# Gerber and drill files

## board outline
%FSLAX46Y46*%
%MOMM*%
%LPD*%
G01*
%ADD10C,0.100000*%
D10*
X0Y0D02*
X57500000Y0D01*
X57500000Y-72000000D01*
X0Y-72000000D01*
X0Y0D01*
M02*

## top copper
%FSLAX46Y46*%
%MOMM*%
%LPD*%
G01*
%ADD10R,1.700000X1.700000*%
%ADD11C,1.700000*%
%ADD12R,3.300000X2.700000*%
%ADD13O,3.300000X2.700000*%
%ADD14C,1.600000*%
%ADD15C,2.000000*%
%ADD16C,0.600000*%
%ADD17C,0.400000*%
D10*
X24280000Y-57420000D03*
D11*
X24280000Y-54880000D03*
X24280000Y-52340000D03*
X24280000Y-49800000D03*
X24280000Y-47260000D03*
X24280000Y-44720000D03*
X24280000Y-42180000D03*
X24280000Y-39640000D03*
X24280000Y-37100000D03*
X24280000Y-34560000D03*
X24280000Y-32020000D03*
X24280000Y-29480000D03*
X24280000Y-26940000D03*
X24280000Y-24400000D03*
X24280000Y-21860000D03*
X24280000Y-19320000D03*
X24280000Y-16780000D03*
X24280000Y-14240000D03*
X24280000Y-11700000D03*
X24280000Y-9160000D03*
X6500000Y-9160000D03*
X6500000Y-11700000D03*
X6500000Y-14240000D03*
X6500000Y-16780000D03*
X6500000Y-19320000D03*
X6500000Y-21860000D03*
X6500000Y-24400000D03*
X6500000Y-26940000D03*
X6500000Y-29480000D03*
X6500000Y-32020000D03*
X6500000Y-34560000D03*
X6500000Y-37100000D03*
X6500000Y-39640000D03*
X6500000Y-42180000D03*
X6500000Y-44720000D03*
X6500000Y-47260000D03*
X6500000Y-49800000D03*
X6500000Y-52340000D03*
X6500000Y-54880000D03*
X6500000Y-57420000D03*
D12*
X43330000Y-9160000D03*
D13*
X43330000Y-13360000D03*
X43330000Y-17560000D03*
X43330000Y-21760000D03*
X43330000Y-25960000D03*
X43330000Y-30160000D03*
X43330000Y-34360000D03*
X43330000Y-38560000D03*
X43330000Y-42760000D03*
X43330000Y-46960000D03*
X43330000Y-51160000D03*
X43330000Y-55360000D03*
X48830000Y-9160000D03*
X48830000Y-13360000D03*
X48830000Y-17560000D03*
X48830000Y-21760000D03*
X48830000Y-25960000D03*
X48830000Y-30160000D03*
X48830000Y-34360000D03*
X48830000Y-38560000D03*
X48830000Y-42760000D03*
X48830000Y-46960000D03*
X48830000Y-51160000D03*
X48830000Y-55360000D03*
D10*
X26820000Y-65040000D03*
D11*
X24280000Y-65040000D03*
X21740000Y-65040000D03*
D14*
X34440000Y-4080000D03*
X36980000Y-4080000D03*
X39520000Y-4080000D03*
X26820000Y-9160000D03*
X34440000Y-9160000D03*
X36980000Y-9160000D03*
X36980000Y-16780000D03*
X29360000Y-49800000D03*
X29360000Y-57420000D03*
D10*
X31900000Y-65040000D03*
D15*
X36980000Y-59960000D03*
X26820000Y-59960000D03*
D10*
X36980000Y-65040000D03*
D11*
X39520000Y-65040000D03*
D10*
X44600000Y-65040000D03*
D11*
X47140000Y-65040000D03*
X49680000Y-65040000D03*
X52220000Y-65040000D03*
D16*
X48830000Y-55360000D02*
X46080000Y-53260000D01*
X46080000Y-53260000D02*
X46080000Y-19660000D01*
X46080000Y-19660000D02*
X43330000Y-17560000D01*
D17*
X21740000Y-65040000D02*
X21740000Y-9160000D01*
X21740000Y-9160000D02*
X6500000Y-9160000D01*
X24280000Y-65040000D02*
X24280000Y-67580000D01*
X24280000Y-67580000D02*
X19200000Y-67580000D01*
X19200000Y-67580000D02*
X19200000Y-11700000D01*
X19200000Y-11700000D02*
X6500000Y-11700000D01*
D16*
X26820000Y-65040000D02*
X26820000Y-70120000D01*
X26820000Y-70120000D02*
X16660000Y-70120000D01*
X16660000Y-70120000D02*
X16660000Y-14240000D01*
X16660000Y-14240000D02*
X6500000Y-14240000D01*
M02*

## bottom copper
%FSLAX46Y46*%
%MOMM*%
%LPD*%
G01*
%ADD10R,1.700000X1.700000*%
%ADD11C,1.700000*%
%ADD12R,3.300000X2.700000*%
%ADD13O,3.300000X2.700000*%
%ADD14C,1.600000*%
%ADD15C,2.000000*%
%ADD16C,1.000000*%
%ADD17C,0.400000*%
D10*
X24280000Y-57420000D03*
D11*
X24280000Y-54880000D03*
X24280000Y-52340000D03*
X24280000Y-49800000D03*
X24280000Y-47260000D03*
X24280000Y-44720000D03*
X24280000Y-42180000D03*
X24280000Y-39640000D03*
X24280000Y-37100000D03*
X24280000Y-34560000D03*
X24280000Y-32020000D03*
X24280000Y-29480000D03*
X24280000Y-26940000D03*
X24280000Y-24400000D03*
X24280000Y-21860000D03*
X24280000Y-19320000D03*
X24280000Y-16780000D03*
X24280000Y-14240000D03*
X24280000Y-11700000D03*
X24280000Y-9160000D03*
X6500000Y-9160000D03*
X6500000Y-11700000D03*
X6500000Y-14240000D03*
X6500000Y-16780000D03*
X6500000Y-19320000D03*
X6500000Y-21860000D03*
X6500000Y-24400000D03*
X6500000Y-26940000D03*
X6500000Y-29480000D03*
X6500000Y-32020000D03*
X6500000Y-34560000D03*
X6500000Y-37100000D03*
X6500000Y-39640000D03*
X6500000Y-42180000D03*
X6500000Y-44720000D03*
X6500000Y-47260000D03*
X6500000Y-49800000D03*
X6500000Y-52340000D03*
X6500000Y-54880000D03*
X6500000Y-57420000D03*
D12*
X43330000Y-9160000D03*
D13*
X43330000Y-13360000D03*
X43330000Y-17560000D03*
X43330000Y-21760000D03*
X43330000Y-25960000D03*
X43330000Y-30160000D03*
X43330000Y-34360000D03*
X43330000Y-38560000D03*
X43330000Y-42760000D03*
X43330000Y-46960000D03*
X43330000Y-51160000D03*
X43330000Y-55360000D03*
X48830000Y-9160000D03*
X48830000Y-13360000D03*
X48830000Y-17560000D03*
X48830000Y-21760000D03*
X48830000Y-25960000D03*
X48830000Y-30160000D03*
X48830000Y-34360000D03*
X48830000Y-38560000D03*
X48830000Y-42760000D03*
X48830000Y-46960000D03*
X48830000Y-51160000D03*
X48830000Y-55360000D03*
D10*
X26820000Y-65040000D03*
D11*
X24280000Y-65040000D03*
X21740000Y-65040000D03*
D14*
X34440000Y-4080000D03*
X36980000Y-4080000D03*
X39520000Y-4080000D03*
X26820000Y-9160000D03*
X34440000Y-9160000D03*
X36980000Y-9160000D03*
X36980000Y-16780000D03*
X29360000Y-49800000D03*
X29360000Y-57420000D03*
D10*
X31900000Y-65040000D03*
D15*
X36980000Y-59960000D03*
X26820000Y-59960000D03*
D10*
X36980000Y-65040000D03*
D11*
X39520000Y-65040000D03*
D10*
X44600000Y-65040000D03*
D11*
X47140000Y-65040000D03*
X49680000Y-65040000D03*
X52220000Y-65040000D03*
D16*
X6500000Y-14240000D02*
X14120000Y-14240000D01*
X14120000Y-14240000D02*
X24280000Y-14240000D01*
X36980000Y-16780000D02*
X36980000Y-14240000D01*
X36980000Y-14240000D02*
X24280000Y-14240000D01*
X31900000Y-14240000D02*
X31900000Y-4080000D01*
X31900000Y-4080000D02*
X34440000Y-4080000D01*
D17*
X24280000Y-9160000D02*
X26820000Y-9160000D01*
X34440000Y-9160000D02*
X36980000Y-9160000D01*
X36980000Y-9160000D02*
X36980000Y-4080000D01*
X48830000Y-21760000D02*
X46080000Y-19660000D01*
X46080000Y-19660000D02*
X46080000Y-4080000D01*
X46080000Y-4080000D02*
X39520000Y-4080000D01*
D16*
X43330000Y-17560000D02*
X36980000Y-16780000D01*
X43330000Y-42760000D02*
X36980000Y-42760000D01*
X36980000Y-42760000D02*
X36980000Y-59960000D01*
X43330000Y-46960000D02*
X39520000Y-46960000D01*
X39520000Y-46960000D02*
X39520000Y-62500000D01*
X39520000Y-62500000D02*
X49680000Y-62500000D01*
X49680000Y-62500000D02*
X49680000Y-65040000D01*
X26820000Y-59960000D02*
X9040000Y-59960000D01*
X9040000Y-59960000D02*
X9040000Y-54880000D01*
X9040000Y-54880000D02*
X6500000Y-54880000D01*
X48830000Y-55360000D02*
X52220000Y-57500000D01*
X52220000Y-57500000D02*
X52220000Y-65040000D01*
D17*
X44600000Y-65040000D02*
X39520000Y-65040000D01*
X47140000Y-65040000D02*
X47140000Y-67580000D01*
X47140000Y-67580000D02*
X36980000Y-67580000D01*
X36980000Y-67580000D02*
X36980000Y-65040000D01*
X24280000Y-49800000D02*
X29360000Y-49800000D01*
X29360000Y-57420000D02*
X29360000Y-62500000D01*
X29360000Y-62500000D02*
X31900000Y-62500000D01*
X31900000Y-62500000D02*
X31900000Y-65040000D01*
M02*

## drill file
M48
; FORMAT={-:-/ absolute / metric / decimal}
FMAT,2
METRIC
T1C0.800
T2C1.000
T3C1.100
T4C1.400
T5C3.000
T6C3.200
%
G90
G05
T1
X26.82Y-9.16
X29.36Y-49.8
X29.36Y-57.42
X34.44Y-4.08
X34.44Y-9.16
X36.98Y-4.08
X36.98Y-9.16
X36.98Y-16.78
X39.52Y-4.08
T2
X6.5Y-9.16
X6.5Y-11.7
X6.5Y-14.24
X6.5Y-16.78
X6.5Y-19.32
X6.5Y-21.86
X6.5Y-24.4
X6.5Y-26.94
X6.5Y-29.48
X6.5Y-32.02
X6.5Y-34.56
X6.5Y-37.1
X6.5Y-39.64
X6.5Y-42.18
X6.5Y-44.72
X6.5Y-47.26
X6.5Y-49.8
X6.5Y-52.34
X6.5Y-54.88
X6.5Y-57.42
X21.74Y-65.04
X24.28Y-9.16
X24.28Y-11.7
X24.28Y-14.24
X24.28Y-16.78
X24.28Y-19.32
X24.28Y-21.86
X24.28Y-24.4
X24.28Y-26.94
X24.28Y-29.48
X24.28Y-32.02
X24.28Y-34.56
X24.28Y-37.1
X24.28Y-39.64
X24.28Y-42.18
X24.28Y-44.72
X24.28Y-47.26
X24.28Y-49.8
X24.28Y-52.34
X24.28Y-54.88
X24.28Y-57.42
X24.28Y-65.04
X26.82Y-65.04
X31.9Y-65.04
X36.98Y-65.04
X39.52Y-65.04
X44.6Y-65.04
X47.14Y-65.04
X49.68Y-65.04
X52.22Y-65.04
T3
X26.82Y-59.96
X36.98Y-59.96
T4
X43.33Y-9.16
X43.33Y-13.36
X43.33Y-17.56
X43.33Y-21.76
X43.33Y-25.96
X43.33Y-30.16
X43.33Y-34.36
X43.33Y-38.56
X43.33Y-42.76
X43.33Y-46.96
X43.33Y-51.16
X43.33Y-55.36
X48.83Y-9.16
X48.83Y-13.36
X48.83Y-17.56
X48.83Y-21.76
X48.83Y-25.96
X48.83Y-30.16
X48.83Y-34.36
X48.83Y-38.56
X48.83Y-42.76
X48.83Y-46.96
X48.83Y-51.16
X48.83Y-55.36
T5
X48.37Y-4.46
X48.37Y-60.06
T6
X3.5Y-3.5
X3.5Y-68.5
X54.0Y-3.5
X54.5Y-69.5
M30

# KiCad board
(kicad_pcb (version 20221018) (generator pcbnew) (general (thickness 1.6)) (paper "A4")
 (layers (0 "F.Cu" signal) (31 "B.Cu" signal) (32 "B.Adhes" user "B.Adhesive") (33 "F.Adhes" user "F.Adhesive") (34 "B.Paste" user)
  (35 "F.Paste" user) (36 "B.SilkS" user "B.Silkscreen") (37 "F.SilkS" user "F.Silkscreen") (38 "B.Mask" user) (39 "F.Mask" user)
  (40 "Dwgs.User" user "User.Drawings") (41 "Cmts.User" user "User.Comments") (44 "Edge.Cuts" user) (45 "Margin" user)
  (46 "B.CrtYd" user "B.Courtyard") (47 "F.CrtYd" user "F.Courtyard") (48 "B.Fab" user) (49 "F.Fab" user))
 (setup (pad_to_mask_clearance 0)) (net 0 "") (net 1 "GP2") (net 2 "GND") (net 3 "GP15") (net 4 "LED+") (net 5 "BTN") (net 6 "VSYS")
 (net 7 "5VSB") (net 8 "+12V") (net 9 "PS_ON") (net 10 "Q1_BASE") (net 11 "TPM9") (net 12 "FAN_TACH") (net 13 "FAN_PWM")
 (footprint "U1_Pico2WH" (layer "F.Cu") (at 15.390 33.290) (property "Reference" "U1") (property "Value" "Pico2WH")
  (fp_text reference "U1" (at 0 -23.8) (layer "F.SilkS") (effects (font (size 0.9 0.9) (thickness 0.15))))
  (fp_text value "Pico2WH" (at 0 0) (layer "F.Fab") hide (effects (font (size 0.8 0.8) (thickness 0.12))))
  (pad "1" thru_hole rect (at 8.890 24.130) (size 1.7 1.7) (drill 1.0) (layers "*.Cu" "*.Mask"))
  (pad "2" thru_hole circle (at 8.890 21.590) (size 1.7 1.7) (drill 1.0) (layers "*.Cu" "*.Mask"))
  (pad "3" thru_hole circle (at 8.890 19.050) (size 1.7 1.7) (drill 1.0) (layers "*.Cu" "*.Mask"))
  (pad "4" thru_hole circle (at 8.890 16.510) (size 1.7 1.7) (drill 1.0) (layers "*.Cu" "*.Mask") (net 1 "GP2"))
  (pad "5" thru_hole circle (at 8.890 13.970) (size 1.7 1.7) (drill 1.0) (layers "*.Cu" "*.Mask"))
  (pad "6" thru_hole circle (at 8.890 11.430) (size 1.7 1.7) (drill 1.0) (layers "*.Cu" "*.Mask"))
  (pad "7" thru_hole circle (at 8.890 8.890) (size 1.7 1.7) (drill 1.0) (layers "*.Cu" "*.Mask"))
  (pad "8" thru_hole circle (at 8.890 6.350) (size 1.7 1.7) (drill 1.0) (layers "*.Cu" "*.Mask"))
  (pad "9" thru_hole circle (at 8.890 3.810) (size 1.7 1.7) (drill 1.0) (layers "*.Cu" "*.Mask"))
  (pad "10" thru_hole circle (at 8.890 1.270) (size 1.7 1.7) (drill 1.0) (layers "*.Cu" "*.Mask"))
  (pad "11" thru_hole circle (at 8.890 -1.270) (size 1.7 1.7) (drill 1.0) (layers "*.Cu" "*.Mask"))
  (pad "12" thru_hole circle (at 8.890 -3.810) (size 1.7 1.7) (drill 1.0) (layers "*.Cu" "*.Mask"))
  (pad "13" thru_hole circle (at 8.890 -6.350) (size 1.7 1.7) (drill 1.0) (layers "*.Cu" "*.Mask"))
  (pad "14" thru_hole circle (at 8.890 -8.890) (size 1.7 1.7) (drill 1.0) (layers "*.Cu" "*.Mask"))
  (pad "15" thru_hole circle (at 8.890 -11.430) (size 1.7 1.7) (drill 1.0) (layers "*.Cu" "*.Mask"))
  (pad "16" thru_hole circle (at 8.890 -13.970) (size 1.7 1.7) (drill 1.0) (layers "*.Cu" "*.Mask"))
  (pad "17" thru_hole circle (at 8.890 -16.510) (size 1.7 1.7) (drill 1.0) (layers "*.Cu" "*.Mask"))
  (pad "18" thru_hole circle (at 8.890 -19.050) (size 1.7 1.7) (drill 1.0) (layers "*.Cu" "*.Mask") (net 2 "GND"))
  (pad "19" thru_hole circle (at 8.890 -21.590) (size 1.7 1.7) (drill 1.0) (layers "*.Cu" "*.Mask"))
  (pad "20" thru_hole circle (at 8.890 -24.130) (size 1.7 1.7) (drill 1.0) (layers "*.Cu" "*.Mask") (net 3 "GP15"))
  (pad "21" thru_hole circle (at -8.890 -24.130) (size 1.7 1.7) (drill 1.0) (layers "*.Cu" "*.Mask") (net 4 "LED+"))
  (pad "22" thru_hole circle (at -8.890 -21.590) (size 1.7 1.7) (drill 1.0) (layers "*.Cu" "*.Mask") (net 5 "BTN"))
  (pad "23" thru_hole circle (at -8.890 -19.050) (size 1.7 1.7) (drill 1.0) (layers "*.Cu" "*.Mask") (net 2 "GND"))
  (pad "24" thru_hole circle (at -8.890 -16.510) (size 1.7 1.7) (drill 1.0) (layers "*.Cu" "*.Mask"))
  (pad "25" thru_hole circle (at -8.890 -13.970) (size 1.7 1.7) (drill 1.0) (layers "*.Cu" "*.Mask"))
  (pad "26" thru_hole circle (at -8.890 -11.430) (size 1.7 1.7) (drill 1.0) (layers "*.Cu" "*.Mask"))
  (pad "27" thru_hole circle (at -8.890 -8.890) (size 1.7 1.7) (drill 1.0) (layers "*.Cu" "*.Mask"))
  (pad "28" thru_hole circle (at -8.890 -6.350) (size 1.7 1.7) (drill 1.0) (layers "*.Cu" "*.Mask"))
  (pad "29" thru_hole circle (at -8.890 -3.810) (size 1.7 1.7) (drill 1.0) (layers "*.Cu" "*.Mask"))
  (pad "30" thru_hole circle (at -8.890 -1.270) (size 1.7 1.7) (drill 1.0) (layers "*.Cu" "*.Mask"))
  (pad "31" thru_hole circle (at -8.890 1.270) (size 1.7 1.7) (drill 1.0) (layers "*.Cu" "*.Mask"))
  (pad "32" thru_hole circle (at -8.890 3.810) (size 1.7 1.7) (drill 1.0) (layers "*.Cu" "*.Mask"))
  (pad "33" thru_hole circle (at -8.890 6.350) (size 1.7 1.7) (drill 1.0) (layers "*.Cu" "*.Mask"))
  (pad "34" thru_hole circle (at -8.890 8.890) (size 1.7 1.7) (drill 1.0) (layers "*.Cu" "*.Mask"))
  (pad "35" thru_hole circle (at -8.890 11.430) (size 1.7 1.7) (drill 1.0) (layers "*.Cu" "*.Mask"))
  (pad "36" thru_hole circle (at -8.890 13.970) (size 1.7 1.7) (drill 1.0) (layers "*.Cu" "*.Mask"))
  (pad "37" thru_hole circle (at -8.890 16.510) (size 1.7 1.7) (drill 1.0) (layers "*.Cu" "*.Mask"))
  (pad "38" thru_hole circle (at -8.890 19.050) (size 1.7 1.7) (drill 1.0) (layers "*.Cu" "*.Mask"))
  (pad "39" thru_hole circle (at -8.890 21.590) (size 1.7 1.7) (drill 1.0) (layers "*.Cu" "*.Mask") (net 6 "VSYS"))
  (pad "40" thru_hole circle (at -8.890 24.130) (size 1.7 1.7) (drill 1.0) (layers "*.Cu" "*.Mask")))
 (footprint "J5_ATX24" (layer "F.Cu") (at 46.080 32.260) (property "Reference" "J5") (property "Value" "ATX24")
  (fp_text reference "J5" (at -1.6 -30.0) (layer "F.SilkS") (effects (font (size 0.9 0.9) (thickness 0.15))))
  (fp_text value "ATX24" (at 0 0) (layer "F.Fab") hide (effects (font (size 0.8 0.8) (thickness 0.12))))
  (pad "1" thru_hole rect (at -2.750 -23.100) (size 3.3 2.7) (drill 1.4) (layers "*.Cu" "*.Mask"))
  (pad "2" thru_hole oval (at -2.750 -18.900) (size 3.3 2.7) (drill 1.4) (layers "*.Cu" "*.Mask"))
  (pad "3" thru_hole oval (at -2.750 -14.700) (size 3.3 2.7) (drill 1.4) (layers "*.Cu" "*.Mask") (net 2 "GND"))
  (pad "4" thru_hole oval (at -2.750 -10.500) (size 3.3 2.7) (drill 1.4) (layers "*.Cu" "*.Mask"))
  (pad "5" thru_hole oval (at -2.750 -6.300) (size 3.3 2.7) (drill 1.4) (layers "*.Cu" "*.Mask"))
  (pad "6" thru_hole oval (at -2.750 -2.100) (size 3.3 2.7) (drill 1.4) (layers "*.Cu" "*.Mask"))
  (pad "7" thru_hole oval (at -2.750 2.100) (size 3.3 2.7) (drill 1.4) (layers "*.Cu" "*.Mask"))
  (pad "8" thru_hole oval (at -2.750 6.300) (size 3.3 2.7) (drill 1.4) (layers "*.Cu" "*.Mask"))
  (pad "9" thru_hole oval (at -2.750 10.500) (size 3.3 2.7) (drill 1.4) (layers "*.Cu" "*.Mask") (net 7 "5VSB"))
  (pad "10" thru_hole oval (at -2.750 14.700) (size 3.3 2.7) (drill 1.4) (layers "*.Cu" "*.Mask") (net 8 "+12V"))
  (pad "11" thru_hole oval (at -2.750 18.900) (size 3.3 2.7) (drill 1.4) (layers "*.Cu" "*.Mask"))
  (pad "12" thru_hole oval (at -2.750 23.100) (size 3.3 2.7) (drill 1.4) (layers "*.Cu" "*.Mask"))
  (pad "13" thru_hole oval (at 2.750 -23.100) (size 3.3 2.7) (drill 1.4) (layers "*.Cu" "*.Mask"))
  (pad "14" thru_hole oval (at 2.750 -18.900) (size 3.3 2.7) (drill 1.4) (layers "*.Cu" "*.Mask"))
  (pad "15" thru_hole oval (at 2.750 -14.700) (size 3.3 2.7) (drill 1.4) (layers "*.Cu" "*.Mask"))
  (pad "16" thru_hole oval (at 2.750 -10.500) (size 3.3 2.7) (drill 1.4) (layers "*.Cu" "*.Mask") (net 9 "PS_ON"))
  (pad "17" thru_hole oval (at 2.750 -6.300) (size 3.3 2.7) (drill 1.4) (layers "*.Cu" "*.Mask"))
  (pad "18" thru_hole oval (at 2.750 -2.100) (size 3.3 2.7) (drill 1.4) (layers "*.Cu" "*.Mask"))
  (pad "19" thru_hole oval (at 2.750 2.100) (size 3.3 2.7) (drill 1.4) (layers "*.Cu" "*.Mask"))
  (pad "20" thru_hole oval (at 2.750 6.300) (size 3.3 2.7) (drill 1.4) (layers "*.Cu" "*.Mask"))
  (pad "21" thru_hole oval (at 2.750 10.500) (size 3.3 2.7) (drill 1.4) (layers "*.Cu" "*.Mask"))
  (pad "22" thru_hole oval (at 2.750 14.700) (size 3.3 2.7) (drill 1.4) (layers "*.Cu" "*.Mask"))
  (pad "23" thru_hole oval (at 2.750 18.900) (size 3.3 2.7) (drill 1.4) (layers "*.Cu" "*.Mask"))
  (pad "24" thru_hole oval (at 2.750 23.100) (size 3.3 2.7) (drill 1.4) (layers "*.Cu" "*.Mask") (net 2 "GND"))
  (pad "" np_thru_hole circle (at 2.290 -27.800) (size 3.0 3.0) (drill 3.0) (layers "*.Cu" "*.Mask"))
  (pad "" np_thru_hole circle (at 2.290 27.800) (size 3.0 3.0) (drill 3.0) (layers "*.Cu" "*.Mask")))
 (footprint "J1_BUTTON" (layer "F.Cu") (at 24.280 65.040) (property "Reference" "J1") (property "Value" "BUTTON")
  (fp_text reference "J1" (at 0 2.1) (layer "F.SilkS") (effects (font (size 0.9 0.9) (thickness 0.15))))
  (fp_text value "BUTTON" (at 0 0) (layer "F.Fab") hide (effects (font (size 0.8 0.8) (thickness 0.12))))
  (pad "1" thru_hole rect (at 2.540 0.000) (size 1.7 1.7) (drill 1.0) (layers "*.Cu" "*.Mask") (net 2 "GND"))
  (pad "2" thru_hole circle (at 0.000 0.000) (size 1.7 1.7) (drill 1.0) (layers "*.Cu" "*.Mask") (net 5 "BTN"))
  (pad "3" thru_hole circle (at -2.540 0.000) (size 1.7 1.7) (drill 1.0) (layers "*.Cu" "*.Mask") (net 4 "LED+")))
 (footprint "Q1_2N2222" (layer "F.Cu") (at 36.980 4.080) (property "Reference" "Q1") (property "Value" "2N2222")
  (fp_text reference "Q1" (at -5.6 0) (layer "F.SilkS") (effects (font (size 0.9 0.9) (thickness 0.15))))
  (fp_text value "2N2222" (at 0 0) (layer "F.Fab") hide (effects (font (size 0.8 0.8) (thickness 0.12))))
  (pad "E" thru_hole circle (at -2.540 0.000) (size 1.6 1.6) (drill 0.8) (layers "*.Cu" "*.Mask") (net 2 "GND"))
  (pad "B" thru_hole circle (at 0.000 0.000) (size 1.6 1.6) (drill 0.8) (layers "*.Cu" "*.Mask") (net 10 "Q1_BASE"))
  (pad "C" thru_hole circle (at 2.540 0.000) (size 1.6 1.6) (drill 0.8) (layers "*.Cu" "*.Mask") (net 9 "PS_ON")))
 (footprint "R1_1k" (layer "F.Cu") (at 30.630 9.160) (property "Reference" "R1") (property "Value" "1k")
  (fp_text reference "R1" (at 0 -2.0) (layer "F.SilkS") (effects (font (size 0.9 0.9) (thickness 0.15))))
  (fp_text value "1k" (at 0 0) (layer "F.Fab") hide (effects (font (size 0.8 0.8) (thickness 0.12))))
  (pad "1" thru_hole circle (at -3.810 0.000) (size 1.6 1.6) (drill 0.8) (layers "*.Cu" "*.Mask") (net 3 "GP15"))
  (pad "2" thru_hole circle (at 3.810 0.000) (size 1.6 1.6) (drill 0.8) (layers "*.Cu" "*.Mask") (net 10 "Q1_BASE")))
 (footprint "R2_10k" (layer "F.Cu") (at 36.980 12.970) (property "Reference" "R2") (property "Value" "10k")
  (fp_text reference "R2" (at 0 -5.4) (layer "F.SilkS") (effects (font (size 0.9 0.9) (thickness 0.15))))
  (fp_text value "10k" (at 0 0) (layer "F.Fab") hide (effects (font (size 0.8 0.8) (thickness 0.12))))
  (pad "1" thru_hole circle (at 0.000 -3.810) (size 1.6 1.6) (drill 0.8) (layers "*.Cu" "*.Mask") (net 10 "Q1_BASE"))
  (pad "2" thru_hole circle (at 0.000 3.810) (size 1.6 1.6) (drill 0.8) (layers "*.Cu" "*.Mask") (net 2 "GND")))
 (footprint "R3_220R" (layer "F.Cu") (at 29.360 53.610) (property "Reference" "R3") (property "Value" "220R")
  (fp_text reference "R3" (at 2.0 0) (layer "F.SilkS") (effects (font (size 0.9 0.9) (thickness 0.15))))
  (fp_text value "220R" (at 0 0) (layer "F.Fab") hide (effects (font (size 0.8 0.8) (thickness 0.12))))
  (pad "1" thru_hole circle (at 0.000 -3.810) (size 1.6 1.6) (drill 0.8) (layers "*.Cu" "*.Mask") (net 1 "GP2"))
  (pad "2" thru_hole circle (at 0.000 3.810) (size 1.6 1.6) (drill 0.8) (layers "*.Cu" "*.Mask") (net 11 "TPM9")))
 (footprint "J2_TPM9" (layer "F.Cu") (at 31.900 65.040) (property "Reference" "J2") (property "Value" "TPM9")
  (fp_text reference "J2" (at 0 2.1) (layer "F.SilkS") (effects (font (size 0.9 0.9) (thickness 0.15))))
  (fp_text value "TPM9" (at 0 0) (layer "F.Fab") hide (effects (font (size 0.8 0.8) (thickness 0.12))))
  (pad "1" thru_hole rect (at 0.000 0.000) (size 1.7 1.7) (drill 1.0) (layers "*.Cu" "*.Mask") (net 11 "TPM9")))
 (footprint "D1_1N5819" (layer "F.Cu") (at 31.900 59.960) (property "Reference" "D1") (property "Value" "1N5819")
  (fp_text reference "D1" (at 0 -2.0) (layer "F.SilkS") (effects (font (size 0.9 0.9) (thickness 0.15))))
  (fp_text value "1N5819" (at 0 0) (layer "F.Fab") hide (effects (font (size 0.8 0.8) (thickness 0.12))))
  (pad "A" thru_hole circle (at 5.080 0.000) (size 2.0 2.0) (drill 1.1) (layers "*.Cu" "*.Mask") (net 7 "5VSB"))
  (pad "K" thru_hole circle (at -5.080 0.000) (size 2.0 2.0) (drill 1.1) (layers "*.Cu" "*.Mask") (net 6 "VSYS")))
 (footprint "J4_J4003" (layer "F.Cu") (at 38.250 65.040) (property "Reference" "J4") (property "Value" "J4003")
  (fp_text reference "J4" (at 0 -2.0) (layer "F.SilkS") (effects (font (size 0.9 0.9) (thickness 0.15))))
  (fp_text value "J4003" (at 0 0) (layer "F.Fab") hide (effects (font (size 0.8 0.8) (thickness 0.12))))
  (pad "1" thru_hole rect (at -1.270 0.000) (size 1.7 1.7) (drill 1.0) (layers "*.Cu" "*.Mask") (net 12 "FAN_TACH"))
  (pad "2" thru_hole circle (at 1.270 0.000) (size 1.7 1.7) (drill 1.0) (layers "*.Cu" "*.Mask") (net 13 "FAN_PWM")))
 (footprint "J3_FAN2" (layer "F.Cu") (at 48.410 65.040) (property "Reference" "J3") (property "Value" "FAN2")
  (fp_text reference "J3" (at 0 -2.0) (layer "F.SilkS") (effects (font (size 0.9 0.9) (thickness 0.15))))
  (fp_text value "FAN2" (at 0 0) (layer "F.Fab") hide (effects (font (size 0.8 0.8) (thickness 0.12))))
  (pad "1" thru_hole rect (at -3.810 0.000) (size 1.7 1.7) (drill 1.0) (layers "*.Cu" "*.Mask") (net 13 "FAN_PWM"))
  (pad "2" thru_hole circle (at -1.270 0.000) (size 1.7 1.7) (drill 1.0) (layers "*.Cu" "*.Mask") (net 12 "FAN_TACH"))
  (pad "3" thru_hole circle (at 1.270 0.000) (size 1.7 1.7) (drill 1.0) (layers "*.Cu" "*.Mask") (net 8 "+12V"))
  (pad "4" thru_hole circle (at 3.810 0.000) (size 1.7 1.7) (drill 1.0) (layers "*.Cu" "*.Mask") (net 2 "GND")))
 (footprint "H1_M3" (layer "F.Cu") (at 3.500 3.500) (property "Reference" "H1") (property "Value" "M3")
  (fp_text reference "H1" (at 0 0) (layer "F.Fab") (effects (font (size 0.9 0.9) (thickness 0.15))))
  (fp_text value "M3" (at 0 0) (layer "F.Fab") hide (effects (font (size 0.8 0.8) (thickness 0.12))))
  (pad "" np_thru_hole circle (at 0.000 0.000) (size 3.2 3.2) (drill 3.2) (layers "*.Cu" "*.Mask")))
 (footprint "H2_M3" (layer "F.Cu") (at 54.000 3.500) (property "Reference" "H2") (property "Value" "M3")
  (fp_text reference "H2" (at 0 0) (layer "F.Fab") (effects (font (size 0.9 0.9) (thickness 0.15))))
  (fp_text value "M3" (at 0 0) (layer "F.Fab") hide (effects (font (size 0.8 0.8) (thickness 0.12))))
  (pad "" np_thru_hole circle (at 0.000 0.000) (size 3.2 3.2) (drill 3.2) (layers "*.Cu" "*.Mask")))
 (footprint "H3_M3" (layer "F.Cu") (at 3.500 68.500) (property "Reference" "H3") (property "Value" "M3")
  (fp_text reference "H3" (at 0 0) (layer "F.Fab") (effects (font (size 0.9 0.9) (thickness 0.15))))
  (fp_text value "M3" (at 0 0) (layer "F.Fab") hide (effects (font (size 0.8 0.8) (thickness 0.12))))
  (pad "" np_thru_hole circle (at 0.000 0.000) (size 3.2 3.2) (drill 3.2) (layers "*.Cu" "*.Mask")))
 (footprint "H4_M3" (layer "F.Cu") (at 54.500 69.500) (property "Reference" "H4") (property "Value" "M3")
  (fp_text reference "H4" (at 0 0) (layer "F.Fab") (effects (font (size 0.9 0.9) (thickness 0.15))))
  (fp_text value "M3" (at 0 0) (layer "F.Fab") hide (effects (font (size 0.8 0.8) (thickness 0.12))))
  (pad "" np_thru_hole circle (at 0.000 0.000) (size 3.2 3.2) (drill 3.2) (layers "*.Cu" "*.Mask")))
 (segment (start 6.500 14.240) (end 14.120 14.240) (width 1.0) (layer "B.Cu") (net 2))
 (segment (start 14.120 14.240) (end 24.280 14.240) (width 1.0) (layer "B.Cu") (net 2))
 (segment (start 36.980 16.780) (end 36.980 14.240) (width 1.0) (layer "B.Cu") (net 2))
 (segment (start 36.980 14.240) (end 24.280 14.240) (width 1.0) (layer "B.Cu") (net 2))
 (segment (start 31.900 14.240) (end 31.900 4.080) (width 1.0) (layer "B.Cu") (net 2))
 (segment (start 31.900 4.080) (end 34.440 4.080) (width 1.0) (layer "B.Cu") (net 2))
 (segment (start 24.280 9.160) (end 26.820 9.160) (width 0.4) (layer "B.Cu") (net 3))
 (segment (start 34.440 9.160) (end 36.980 9.160) (width 0.4) (layer "B.Cu") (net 10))
 (segment (start 36.980 9.160) (end 36.980 4.080) (width 0.4) (layer "B.Cu") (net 10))
 (segment (start 48.830 21.760) (end 46.080 19.660) (width 0.4) (layer "B.Cu") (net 9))
 (segment (start 46.080 19.660) (end 46.080 4.080) (width 0.4) (layer "B.Cu") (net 9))
 (segment (start 46.080 4.080) (end 39.520 4.080) (width 0.4) (layer "B.Cu") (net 9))
 (segment (start 43.330 17.560) (end 36.980 16.780) (width 1.0) (layer "B.Cu") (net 2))
 (segment (start 43.330 42.760) (end 36.980 42.760) (width 1.0) (layer "B.Cu") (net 7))
 (segment (start 36.980 42.760) (end 36.980 59.960) (width 1.0) (layer "B.Cu") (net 7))
 (segment (start 43.330 46.960) (end 39.520 46.960) (width 1.0) (layer "B.Cu") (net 8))
 (segment (start 39.520 46.960) (end 39.520 62.500) (width 1.0) (layer "B.Cu") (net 8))
 (segment (start 39.520 62.500) (end 49.680 62.500) (width 1.0) (layer "B.Cu") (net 8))
 (segment (start 49.680 62.500) (end 49.680 65.040) (width 1.0) (layer "B.Cu") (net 8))
 (segment (start 26.820 59.960) (end 9.040 59.960) (width 1.0) (layer "B.Cu") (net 6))
 (segment (start 9.040 59.960) (end 9.040 54.880) (width 1.0) (layer "B.Cu") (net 6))
 (segment (start 9.040 54.880) (end 6.500 54.880) (width 1.0) (layer "B.Cu") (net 6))
 (segment (start 48.830 55.360) (end 52.220 57.500) (width 1.0) (layer "B.Cu") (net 2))
 (segment (start 52.220 57.500) (end 52.220 65.040) (width 1.0) (layer "B.Cu") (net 2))
 (segment (start 44.600 65.040) (end 39.520 65.040) (width 0.4) (layer "B.Cu") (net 13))
 (segment (start 47.140 65.040) (end 47.140 67.580) (width 0.4) (layer "B.Cu") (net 12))
 (segment (start 47.140 67.580) (end 36.980 67.580) (width 0.4) (layer "B.Cu") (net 12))
 (segment (start 36.980 67.580) (end 36.980 65.040) (width 0.4) (layer "B.Cu") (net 12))
 (segment (start 24.280 49.800) (end 29.360 49.800) (width 0.4) (layer "B.Cu") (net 1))
 (segment (start 29.360 57.420) (end 29.360 62.500) (width 0.4) (layer "B.Cu") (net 11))
 (segment (start 29.360 62.500) (end 31.900 62.500) (width 0.4) (layer "B.Cu") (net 11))
 (segment (start 31.900 62.500) (end 31.900 65.040) (width 0.4) (layer "B.Cu") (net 11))
 (segment (start 48.830 55.360) (end 46.080 53.260) (width 0.6) (layer "F.Cu") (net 2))
 (segment (start 46.080 53.260) (end 46.080 19.660) (width 0.6) (layer "F.Cu") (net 2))
 (segment (start 46.080 19.660) (end 43.330 17.560) (width 0.6) (layer "F.Cu") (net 2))
 (segment (start 21.740 65.040) (end 21.740 9.160) (width 0.4) (layer "F.Cu") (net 4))
 (segment (start 21.740 9.160) (end 6.500 9.160) (width 0.4) (layer "F.Cu") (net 4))
 (segment (start 24.280 65.040) (end 24.280 67.580) (width 0.4) (layer "F.Cu") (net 5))
 (segment (start 24.280 67.580) (end 19.200 67.580) (width 0.4) (layer "F.Cu") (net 5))
 (segment (start 19.200 67.580) (end 19.200 11.700) (width 0.4) (layer "F.Cu") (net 5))
 (segment (start 19.200 11.700) (end 6.500 11.700) (width 0.4) (layer "F.Cu") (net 5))
 (segment (start 26.820 65.040) (end 26.820 70.120) (width 0.6) (layer "F.Cu") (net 2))
 (segment (start 26.820 70.120) (end 16.660 70.120) (width 0.6) (layer "F.Cu") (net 2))
 (segment (start 16.660 70.120) (end 16.660 14.240) (width 0.6) (layer "F.Cu") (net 2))
 (segment (start 16.660 14.240) (end 6.500 14.240) (width 0.6) (layer "F.Cu") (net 2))
 (gr_rect (start 0 0) (end 57.5 72.0) (stroke (width 0.1) (type solid)) (fill none) (layer "Edge.Cuts")))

